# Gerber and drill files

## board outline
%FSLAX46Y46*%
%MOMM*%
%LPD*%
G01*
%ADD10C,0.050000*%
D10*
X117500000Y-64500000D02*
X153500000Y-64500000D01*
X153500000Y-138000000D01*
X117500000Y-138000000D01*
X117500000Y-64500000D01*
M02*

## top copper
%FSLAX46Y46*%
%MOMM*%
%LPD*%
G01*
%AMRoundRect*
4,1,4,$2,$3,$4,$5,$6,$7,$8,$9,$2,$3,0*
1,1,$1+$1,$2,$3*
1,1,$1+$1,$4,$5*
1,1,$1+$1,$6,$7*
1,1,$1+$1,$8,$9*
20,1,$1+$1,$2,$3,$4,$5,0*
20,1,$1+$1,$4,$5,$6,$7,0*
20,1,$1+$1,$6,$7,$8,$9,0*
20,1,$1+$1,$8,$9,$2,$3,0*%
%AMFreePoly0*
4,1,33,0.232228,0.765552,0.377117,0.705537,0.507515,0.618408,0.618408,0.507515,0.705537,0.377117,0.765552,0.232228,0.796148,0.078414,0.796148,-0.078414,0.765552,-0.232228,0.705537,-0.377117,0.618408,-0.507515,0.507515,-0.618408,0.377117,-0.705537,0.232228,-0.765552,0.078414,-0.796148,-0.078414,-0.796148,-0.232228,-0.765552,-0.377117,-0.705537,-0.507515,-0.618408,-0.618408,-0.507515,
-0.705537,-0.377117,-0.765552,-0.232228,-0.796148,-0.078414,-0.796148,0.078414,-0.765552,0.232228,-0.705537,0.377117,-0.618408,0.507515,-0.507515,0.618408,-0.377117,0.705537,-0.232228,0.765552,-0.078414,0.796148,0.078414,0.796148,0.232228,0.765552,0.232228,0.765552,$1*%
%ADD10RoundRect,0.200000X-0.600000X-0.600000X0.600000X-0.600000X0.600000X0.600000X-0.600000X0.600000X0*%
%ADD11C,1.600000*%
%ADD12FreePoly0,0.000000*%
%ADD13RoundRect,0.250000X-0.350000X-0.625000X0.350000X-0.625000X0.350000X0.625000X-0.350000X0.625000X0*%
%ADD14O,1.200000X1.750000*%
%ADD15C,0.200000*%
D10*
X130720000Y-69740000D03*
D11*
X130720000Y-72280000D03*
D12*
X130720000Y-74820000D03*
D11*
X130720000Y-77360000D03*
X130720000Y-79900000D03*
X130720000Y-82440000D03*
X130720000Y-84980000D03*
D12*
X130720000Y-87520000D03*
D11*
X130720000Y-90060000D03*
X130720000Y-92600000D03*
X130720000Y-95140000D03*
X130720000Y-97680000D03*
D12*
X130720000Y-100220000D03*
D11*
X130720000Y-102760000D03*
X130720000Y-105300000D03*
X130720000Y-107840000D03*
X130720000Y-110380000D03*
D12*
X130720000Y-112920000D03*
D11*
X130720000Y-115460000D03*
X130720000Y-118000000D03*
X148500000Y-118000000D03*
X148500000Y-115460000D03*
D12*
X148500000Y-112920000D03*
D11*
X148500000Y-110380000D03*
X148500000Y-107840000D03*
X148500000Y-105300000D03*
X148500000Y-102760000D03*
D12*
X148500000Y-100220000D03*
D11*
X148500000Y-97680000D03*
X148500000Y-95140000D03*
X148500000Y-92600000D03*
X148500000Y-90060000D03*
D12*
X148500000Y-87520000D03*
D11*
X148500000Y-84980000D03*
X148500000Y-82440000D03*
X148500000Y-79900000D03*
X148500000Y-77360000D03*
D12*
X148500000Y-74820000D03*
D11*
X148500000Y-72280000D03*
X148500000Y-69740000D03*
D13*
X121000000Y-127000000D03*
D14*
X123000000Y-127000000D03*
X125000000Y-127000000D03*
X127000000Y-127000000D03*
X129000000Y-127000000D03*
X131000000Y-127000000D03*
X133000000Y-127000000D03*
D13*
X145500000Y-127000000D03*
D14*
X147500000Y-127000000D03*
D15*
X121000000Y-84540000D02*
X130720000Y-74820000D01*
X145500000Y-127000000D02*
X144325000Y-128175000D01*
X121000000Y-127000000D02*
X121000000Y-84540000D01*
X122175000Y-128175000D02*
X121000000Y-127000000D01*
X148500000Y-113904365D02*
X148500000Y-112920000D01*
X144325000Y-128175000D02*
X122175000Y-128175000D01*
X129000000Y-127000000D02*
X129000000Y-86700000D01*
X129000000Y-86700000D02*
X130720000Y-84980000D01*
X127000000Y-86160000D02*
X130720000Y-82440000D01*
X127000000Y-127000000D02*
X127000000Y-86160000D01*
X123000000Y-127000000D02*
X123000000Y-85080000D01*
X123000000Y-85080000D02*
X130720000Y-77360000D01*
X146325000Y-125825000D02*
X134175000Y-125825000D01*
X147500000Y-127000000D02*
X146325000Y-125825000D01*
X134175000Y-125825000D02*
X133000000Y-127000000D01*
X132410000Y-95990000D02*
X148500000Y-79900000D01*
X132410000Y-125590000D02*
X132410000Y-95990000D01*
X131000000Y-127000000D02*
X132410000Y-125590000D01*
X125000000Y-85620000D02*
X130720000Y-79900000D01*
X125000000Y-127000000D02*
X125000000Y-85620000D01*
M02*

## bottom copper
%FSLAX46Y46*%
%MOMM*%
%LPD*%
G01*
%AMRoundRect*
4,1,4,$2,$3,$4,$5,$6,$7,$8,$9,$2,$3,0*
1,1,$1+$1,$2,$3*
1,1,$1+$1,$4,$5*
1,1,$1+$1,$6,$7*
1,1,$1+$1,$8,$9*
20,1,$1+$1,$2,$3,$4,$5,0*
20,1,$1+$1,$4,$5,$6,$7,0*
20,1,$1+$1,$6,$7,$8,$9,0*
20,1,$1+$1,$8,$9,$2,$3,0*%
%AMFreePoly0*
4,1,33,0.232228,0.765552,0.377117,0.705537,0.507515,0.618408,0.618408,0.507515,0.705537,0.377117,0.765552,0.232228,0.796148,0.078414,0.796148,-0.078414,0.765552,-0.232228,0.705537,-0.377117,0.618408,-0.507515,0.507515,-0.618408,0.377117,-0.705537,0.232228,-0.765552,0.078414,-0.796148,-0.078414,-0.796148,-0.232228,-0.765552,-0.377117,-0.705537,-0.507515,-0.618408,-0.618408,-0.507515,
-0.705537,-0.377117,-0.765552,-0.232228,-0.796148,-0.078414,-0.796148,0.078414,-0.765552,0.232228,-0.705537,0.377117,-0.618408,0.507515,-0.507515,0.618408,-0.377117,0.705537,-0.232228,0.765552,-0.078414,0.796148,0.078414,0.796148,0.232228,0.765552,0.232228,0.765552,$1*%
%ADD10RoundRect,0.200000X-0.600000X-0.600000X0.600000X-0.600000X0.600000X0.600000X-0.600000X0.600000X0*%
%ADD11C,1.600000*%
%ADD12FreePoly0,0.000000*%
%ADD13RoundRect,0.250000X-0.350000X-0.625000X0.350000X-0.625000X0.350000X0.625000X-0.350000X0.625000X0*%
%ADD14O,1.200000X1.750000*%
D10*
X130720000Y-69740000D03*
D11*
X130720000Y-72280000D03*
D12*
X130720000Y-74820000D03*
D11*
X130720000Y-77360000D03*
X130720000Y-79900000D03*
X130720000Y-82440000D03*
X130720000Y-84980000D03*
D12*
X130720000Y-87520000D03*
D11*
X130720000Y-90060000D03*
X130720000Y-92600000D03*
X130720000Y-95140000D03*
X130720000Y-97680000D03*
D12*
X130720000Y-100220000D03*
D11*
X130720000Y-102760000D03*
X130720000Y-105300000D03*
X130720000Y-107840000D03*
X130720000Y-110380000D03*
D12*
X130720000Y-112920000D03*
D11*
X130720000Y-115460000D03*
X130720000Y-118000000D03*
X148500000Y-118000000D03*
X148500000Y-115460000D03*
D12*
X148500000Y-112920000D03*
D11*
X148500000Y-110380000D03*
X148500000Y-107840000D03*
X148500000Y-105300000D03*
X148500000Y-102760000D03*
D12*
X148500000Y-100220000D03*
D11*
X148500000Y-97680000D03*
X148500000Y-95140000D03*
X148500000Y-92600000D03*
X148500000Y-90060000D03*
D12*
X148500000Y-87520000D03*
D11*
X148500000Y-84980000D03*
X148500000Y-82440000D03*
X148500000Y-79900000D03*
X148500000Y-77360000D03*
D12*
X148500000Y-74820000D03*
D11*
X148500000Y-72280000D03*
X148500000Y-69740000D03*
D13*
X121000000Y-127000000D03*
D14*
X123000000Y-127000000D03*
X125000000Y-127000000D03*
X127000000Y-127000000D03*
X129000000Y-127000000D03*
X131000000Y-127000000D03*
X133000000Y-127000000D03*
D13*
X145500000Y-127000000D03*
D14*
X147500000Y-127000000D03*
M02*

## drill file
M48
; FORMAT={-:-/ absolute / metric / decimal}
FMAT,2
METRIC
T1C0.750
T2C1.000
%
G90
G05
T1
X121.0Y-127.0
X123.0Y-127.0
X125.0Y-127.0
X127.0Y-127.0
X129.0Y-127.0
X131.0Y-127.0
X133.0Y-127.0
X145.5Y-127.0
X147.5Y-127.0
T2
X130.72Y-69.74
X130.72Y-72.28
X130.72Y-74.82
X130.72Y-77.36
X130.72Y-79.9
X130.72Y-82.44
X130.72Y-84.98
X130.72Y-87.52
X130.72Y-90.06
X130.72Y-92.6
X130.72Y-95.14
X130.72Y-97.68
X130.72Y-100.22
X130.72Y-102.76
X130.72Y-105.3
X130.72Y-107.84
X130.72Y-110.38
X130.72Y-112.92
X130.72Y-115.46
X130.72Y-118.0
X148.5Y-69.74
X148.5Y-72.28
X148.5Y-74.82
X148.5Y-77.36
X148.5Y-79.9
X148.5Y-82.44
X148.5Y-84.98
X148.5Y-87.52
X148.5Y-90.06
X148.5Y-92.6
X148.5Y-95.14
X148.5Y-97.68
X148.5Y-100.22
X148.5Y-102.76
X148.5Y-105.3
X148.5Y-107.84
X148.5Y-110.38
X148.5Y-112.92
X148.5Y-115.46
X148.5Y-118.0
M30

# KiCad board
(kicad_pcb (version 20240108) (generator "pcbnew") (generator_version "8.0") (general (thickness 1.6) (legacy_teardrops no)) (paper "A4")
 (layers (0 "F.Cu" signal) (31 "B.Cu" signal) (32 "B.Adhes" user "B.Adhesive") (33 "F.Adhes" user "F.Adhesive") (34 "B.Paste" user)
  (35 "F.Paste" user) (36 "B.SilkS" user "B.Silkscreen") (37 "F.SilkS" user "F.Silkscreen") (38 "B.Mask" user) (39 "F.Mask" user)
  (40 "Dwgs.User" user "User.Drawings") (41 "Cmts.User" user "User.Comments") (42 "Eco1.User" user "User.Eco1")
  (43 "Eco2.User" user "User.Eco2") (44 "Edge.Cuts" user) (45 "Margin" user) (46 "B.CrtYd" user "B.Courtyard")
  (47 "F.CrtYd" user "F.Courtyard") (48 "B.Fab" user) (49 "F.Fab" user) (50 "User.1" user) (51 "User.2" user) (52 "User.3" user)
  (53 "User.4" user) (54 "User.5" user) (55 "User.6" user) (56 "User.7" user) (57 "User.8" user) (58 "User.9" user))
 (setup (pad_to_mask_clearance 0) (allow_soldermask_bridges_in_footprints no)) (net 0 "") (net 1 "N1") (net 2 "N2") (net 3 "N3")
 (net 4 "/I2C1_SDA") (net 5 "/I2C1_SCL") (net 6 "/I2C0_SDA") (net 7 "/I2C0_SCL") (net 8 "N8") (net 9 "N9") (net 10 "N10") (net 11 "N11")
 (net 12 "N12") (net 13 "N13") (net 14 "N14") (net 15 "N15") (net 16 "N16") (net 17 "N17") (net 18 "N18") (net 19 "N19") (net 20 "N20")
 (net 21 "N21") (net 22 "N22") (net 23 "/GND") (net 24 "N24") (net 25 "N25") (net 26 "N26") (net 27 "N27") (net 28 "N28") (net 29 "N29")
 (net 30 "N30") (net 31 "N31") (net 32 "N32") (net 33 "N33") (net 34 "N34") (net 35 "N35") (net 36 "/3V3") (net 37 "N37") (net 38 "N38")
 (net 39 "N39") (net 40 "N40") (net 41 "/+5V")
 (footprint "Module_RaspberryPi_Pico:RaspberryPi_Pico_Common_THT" (layer "F.Cu") (at 139.61 93.87)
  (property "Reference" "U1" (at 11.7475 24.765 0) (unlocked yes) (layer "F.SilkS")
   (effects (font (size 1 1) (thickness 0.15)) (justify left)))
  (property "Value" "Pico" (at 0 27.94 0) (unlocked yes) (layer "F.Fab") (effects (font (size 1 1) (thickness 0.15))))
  (pad "1" thru_hole roundrect (at -8.89 -24.13) (size 1.6 1.6) (drill 1) (layers "*.Cu" "*.Mask") (remove_unused_layers no)
   (roundrect_rratio 0.125) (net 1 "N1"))
  (pad "2" thru_hole circle (at -8.89 -21.59) (size 1.6 1.6) (drill 1) (layers "*.Cu" "*.Mask") (remove_unused_layers no) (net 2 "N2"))
  (pad "3" thru_hole custom (at -8.89 -19.05) (size 1.6 1.6) (drill 1) (layers "*.Cu" "*.Mask") (remove_unused_layers no) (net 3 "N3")
   (options (clearance outline) (anchor circle)) (primitives))
  (pad "4" thru_hole circle (at -8.89 -16.51) (size 1.6 1.6) (drill 1) (layers "*.Cu" "*.Mask") (remove_unused_layers no)
   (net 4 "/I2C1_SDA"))
  (pad "5" thru_hole circle (at -8.89 -13.97) (size 1.6 1.6) (drill 1) (layers "*.Cu" "*.Mask") (remove_unused_layers no)
   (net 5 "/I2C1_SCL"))
  (pad "6" thru_hole circle (at -8.89 -11.43) (size 1.6 1.6) (drill 1) (layers "*.Cu" "*.Mask") (remove_unused_layers no)
   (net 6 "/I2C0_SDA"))
  (pad "7" thru_hole circle (at -8.89 -8.89) (size 1.6 1.6) (drill 1) (layers "*.Cu" "*.Mask") (remove_unused_layers no) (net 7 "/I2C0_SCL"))
  (pad "8" thru_hole custom (at -8.89 -6.35) (size 1.6 1.6) (drill 1) (layers "*.Cu" "*.Mask") (remove_unused_layers no) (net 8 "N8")
   (options (clearance outline) (anchor circle)) (primitives))
  (pad "9" thru_hole circle (at -8.89 -3.81) (size 1.6 1.6) (drill 1) (layers "*.Cu" "*.Mask") (remove_unused_layers no) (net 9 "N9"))
  (pad "10" thru_hole circle (at -8.89 -1.27) (size 1.6 1.6) (drill 1) (layers "*.Cu" "*.Mask") (remove_unused_layers no) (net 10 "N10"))
  (pad "11" thru_hole circle (at -8.89 1.27) (size 1.6 1.6) (drill 1) (layers "*.Cu" "*.Mask") (remove_unused_layers no) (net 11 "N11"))
  (pad "12" thru_hole circle (at -8.89 3.81) (size 1.6 1.6) (drill 1) (layers "*.Cu" "*.Mask") (remove_unused_layers no) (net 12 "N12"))
  (pad "13" thru_hole custom (at -8.89 6.35) (size 1.6 1.6) (drill 1) (layers "*.Cu" "*.Mask") (remove_unused_layers no) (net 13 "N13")
   (options (clearance outline) (anchor circle)) (primitives))
  (pad "14" thru_hole circle (at -8.89 8.89) (size 1.6 1.6) (drill 1) (layers "*.Cu" "*.Mask") (remove_unused_layers no) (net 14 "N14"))
  (pad "15" thru_hole circle (at -8.89 11.43) (size 1.6 1.6) (drill 1) (layers "*.Cu" "*.Mask") (remove_unused_layers no) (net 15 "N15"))
  (pad "16" thru_hole circle (at -8.89 13.97) (size 1.6 1.6) (drill 1) (layers "*.Cu" "*.Mask") (remove_unused_layers no) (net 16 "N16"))
  (pad "17" thru_hole circle (at -8.89 16.51) (size 1.6 1.6) (drill 1) (layers "*.Cu" "*.Mask") (remove_unused_layers no) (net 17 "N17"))
  (pad "18" thru_hole custom (at -8.89 19.05) (size 1.6 1.6) (drill 1) (layers "*.Cu" "*.Mask") (remove_unused_layers no) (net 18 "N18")
   (options (clearance outline) (anchor circle)) (primitives))
  (pad "19" thru_hole circle (at -8.89 21.59) (size 1.6 1.6) (drill 1) (layers "*.Cu" "*.Mask") (remove_unused_layers no) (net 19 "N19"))
  (pad "20" thru_hole circle (at -8.89 24.13) (size 1.6 1.6) (drill 1) (layers "*.Cu" "*.Mask") (remove_unused_layers no) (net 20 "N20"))
  (pad "21" thru_hole circle (at 8.89 24.13) (size 1.6 1.6) (drill 1) (layers "*.Cu" "*.Mask") (remove_unused_layers no) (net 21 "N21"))
  (pad "22" thru_hole circle (at 8.89 21.59) (size 1.6 1.6) (drill 1) (layers "*.Cu" "*.Mask") (remove_unused_layers no) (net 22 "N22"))
  (pad "23" thru_hole custom (at 8.89 19.05) (size 1.6 1.6) (drill 1) (layers "*.Cu" "*.Mask") (remove_unused_layers no) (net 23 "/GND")
   (options (clearance outline) (anchor circle)) (primitives))
  (pad "24" thru_hole circle (at 8.89 16.51) (size 1.6 1.6) (drill 1) (layers "*.Cu" "*.Mask") (remove_unused_layers no) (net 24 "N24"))
  (pad "25" thru_hole circle (at 8.89 13.97) (size 1.6 1.6) (drill 1) (layers "*.Cu" "*.Mask") (remove_unused_layers no) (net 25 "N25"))
  (pad "26" thru_hole circle (at 8.89 11.43) (size 1.6 1.6) (drill 1) (layers "*.Cu" "*.Mask") (remove_unused_layers no) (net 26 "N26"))
  (pad "27" thru_hole circle (at 8.89 8.89) (size 1.6 1.6) (drill 1) (layers "*.Cu" "*.Mask") (remove_unused_layers no) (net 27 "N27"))
  (pad "28" thru_hole custom (at 8.89 6.35) (size 1.6 1.6) (drill 1) (layers "*.Cu" "*.Mask") (remove_unused_layers no) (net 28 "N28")
   (options (clearance outline) (anchor circle)) (primitives))
  (pad "29" thru_hole circle (at 8.89 3.81) (size 1.6 1.6) (drill 1) (layers "*.Cu" "*.Mask") (remove_unused_layers no) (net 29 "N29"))
  (pad "30" thru_hole circle (at 8.89 1.27) (size 1.6 1.6) (drill 1) (layers "*.Cu" "*.Mask") (remove_unused_layers no) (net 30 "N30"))
  (pad "31" thru_hole circle (at 8.89 -1.27) (size 1.6 1.6) (drill 1) (layers "*.Cu" "*.Mask") (remove_unused_layers no) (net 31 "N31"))
  (pad "32" thru_hole circle (at 8.89 -3.81) (size 1.6 1.6) (drill 1) (layers "*.Cu" "*.Mask") (remove_unused_layers no) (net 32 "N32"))
  (pad "33" thru_hole custom (at 8.89 -6.35) (size 1.6 1.6) (drill 1) (layers "*.Cu" "*.Mask") (remove_unused_layers no) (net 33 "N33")
   (options (clearance outline) (anchor circle)) (primitives))
  (pad "34" thru_hole circle (at 8.89 -8.89) (size 1.6 1.6) (drill 1) (layers "*.Cu" "*.Mask") (remove_unused_layers no) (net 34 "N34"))
  (pad "35" thru_hole circle (at 8.89 -11.43) (size 1.6 1.6) (drill 1) (layers "*.Cu" "*.Mask") (remove_unused_layers no) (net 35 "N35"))
  (pad "36" thru_hole circle (at 8.89 -13.97) (size 1.6 1.6) (drill 1) (layers "*.Cu" "*.Mask") (remove_unused_layers no) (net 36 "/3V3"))
  (pad "37" thru_hole circle (at 8.89 -16.51) (size 1.6 1.6) (drill 1) (layers "*.Cu" "*.Mask") (remove_unused_layers no) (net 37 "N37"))
  (pad "38" thru_hole custom (at 8.89 -19.05) (size 1.6 1.6) (drill 1) (layers "*.Cu" "*.Mask") (remove_unused_layers no) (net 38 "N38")
   (options (clearance outline) (anchor circle)) (primitives))
  (pad "39" thru_hole circle (at 8.89 -21.59) (size 1.6 1.6) (drill 1) (layers "*.Cu" "*.Mask") (remove_unused_layers no) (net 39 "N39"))
  (pad "40" thru_hole circle (at 8.89 -24.13) (size 1.6 1.6) (drill 1) (layers "*.Cu" "*.Mask") (remove_unused_layers no) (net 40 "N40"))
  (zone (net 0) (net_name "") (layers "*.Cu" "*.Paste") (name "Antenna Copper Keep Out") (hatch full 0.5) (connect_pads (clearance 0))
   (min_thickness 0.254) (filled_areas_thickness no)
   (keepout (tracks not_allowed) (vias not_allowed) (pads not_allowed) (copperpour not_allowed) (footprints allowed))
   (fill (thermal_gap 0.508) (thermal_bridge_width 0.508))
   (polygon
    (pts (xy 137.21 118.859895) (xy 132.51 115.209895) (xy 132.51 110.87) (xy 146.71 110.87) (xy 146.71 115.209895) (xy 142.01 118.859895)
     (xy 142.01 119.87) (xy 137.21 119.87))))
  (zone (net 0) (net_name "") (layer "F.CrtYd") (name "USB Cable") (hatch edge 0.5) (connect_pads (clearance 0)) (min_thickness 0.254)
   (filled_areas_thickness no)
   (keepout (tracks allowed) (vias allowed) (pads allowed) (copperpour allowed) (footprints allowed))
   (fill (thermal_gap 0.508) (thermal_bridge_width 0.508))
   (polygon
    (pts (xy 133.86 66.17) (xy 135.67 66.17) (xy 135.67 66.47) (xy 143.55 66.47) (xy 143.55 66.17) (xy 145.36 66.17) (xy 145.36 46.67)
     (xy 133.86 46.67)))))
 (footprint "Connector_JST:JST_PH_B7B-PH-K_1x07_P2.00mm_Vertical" (layer "F.Cu") (at 121 127)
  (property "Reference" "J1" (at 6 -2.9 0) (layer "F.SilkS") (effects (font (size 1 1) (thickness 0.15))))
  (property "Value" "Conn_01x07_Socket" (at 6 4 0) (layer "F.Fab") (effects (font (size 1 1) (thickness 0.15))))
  (pad "1" thru_hole roundrect (at 0 0) (size 1.2 1.75) (drill 0.75) (layers "*.Cu" "*.Mask") (remove_unused_layers no)
   (roundrect_rratio 0.208333) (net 23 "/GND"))
  (pad "2" thru_hole oval (at 2 0) (size 1.2 1.75) (drill 0.75) (layers "*.Cu" "*.Mask") (remove_unused_layers no) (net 4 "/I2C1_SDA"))
  (pad "3" thru_hole oval (at 4 0) (size 1.2 1.75) (drill 0.75) (layers "*.Cu" "*.Mask") (remove_unused_layers no) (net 5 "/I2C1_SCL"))
  (pad "4" thru_hole oval (at 6 0) (size 1.2 1.75) (drill 0.75) (layers "*.Cu" "*.Mask") (remove_unused_layers no) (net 6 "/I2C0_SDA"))
  (pad "5" thru_hole oval (at 8 0) (size 1.2 1.75) (drill 0.75) (layers "*.Cu" "*.Mask") (remove_unused_layers no) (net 7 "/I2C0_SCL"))
  (pad "6" thru_hole oval (at 10 0) (size 1.2 1.75) (drill 0.75) (layers "*.Cu" "*.Mask") (remove_unused_layers no) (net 36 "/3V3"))
  (pad "7" thru_hole oval (at 12 0) (size 1.2 1.75) (drill 0.75) (layers "*.Cu" "*.Mask") (remove_unused_layers no) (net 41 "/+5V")))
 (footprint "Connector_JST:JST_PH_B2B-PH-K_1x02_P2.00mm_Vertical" (layer "F.Cu") (at 145.5 127)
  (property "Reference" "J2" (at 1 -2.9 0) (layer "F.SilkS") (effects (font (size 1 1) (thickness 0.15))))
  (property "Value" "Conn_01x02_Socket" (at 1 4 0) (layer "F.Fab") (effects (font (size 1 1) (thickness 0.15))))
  (pad "1" thru_hole roundrect (at 0 0) (size 1.2 1.75) (drill 0.75) (layers "*.Cu" "*.Mask") (remove_unused_layers no)
   (roundrect_rratio 0.208333) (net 23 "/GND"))
  (pad "2" thru_hole oval (at 2 0) (size 1.2 1.75) (drill 0.75) (layers "*.Cu" "*.Mask") (remove_unused_layers no) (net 41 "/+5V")))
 (gr_rect (start 117.5 64.5) (end 153.5 138) (stroke (width 0.05) (type default)) (fill none) (layer "Edge.Cuts"))
 (segment (start 121 84.54) (end 130.72 74.82) (width 0.2) (layer "F.Cu") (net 23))
 (segment (start 145.5 127) (end 144.325 128.175) (width 0.2) (layer "F.Cu") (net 23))
 (segment (start 121 127) (end 121 84.54) (width 0.2) (layer "F.Cu") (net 23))
 (segment (start 122.175 128.175) (end 121 127) (width 0.2) (layer "F.Cu") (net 23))
 (segment (start 148.5 113.904365) (end 148.5 112.92) (width 0.2) (layer "F.Cu") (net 23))
 (segment (start 144.325 128.175) (end 122.175 128.175) (width 0.2) (layer "F.Cu") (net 23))
 (segment (start 129 127) (end 129 86.7) (width 0.2) (layer "F.Cu") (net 7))
 (segment (start 129 86.7) (end 130.72 84.98) (width 0.2) (layer "F.Cu") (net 7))
 (segment (start 127 86.16) (end 130.72 82.44) (width 0.2) (layer "F.Cu") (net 6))
 (segment (start 127 127) (end 127 86.16) (width 0.2) (layer "F.Cu") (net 6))
 (segment (start 123 127) (end 123 85.08) (width 0.2) (layer "F.Cu") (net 4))
 (segment (start 123 85.08) (end 130.72 77.36) (width 0.2) (layer "F.Cu") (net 4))
 (segment (start 146.325 125.825) (end 134.175 125.825) (width 0.2) (layer "F.Cu") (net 41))
 (segment (start 147.5 127) (end 146.325 125.825) (width 0.2) (layer "F.Cu") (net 41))
 (segment (start 134.175 125.825) (end 133 127) (width 0.2) (layer "F.Cu") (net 41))
 (segment (start 132.41 95.99) (end 148.5 79.9) (width 0.2) (layer "F.Cu") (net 36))
 (segment (start 132.41 125.59) (end 132.41 95.99) (width 0.2) (layer "F.Cu") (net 36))
 (segment (start 131 127) (end 132.41 125.59) (width 0.2) (layer "F.Cu") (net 36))
 (segment (start 125 85.62) (end 130.72 79.9) (width 0.2) (layer "F.Cu") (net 5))
 (segment (start 125 127) (end 125 85.62) (width 0.2) (layer "F.Cu") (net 5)))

